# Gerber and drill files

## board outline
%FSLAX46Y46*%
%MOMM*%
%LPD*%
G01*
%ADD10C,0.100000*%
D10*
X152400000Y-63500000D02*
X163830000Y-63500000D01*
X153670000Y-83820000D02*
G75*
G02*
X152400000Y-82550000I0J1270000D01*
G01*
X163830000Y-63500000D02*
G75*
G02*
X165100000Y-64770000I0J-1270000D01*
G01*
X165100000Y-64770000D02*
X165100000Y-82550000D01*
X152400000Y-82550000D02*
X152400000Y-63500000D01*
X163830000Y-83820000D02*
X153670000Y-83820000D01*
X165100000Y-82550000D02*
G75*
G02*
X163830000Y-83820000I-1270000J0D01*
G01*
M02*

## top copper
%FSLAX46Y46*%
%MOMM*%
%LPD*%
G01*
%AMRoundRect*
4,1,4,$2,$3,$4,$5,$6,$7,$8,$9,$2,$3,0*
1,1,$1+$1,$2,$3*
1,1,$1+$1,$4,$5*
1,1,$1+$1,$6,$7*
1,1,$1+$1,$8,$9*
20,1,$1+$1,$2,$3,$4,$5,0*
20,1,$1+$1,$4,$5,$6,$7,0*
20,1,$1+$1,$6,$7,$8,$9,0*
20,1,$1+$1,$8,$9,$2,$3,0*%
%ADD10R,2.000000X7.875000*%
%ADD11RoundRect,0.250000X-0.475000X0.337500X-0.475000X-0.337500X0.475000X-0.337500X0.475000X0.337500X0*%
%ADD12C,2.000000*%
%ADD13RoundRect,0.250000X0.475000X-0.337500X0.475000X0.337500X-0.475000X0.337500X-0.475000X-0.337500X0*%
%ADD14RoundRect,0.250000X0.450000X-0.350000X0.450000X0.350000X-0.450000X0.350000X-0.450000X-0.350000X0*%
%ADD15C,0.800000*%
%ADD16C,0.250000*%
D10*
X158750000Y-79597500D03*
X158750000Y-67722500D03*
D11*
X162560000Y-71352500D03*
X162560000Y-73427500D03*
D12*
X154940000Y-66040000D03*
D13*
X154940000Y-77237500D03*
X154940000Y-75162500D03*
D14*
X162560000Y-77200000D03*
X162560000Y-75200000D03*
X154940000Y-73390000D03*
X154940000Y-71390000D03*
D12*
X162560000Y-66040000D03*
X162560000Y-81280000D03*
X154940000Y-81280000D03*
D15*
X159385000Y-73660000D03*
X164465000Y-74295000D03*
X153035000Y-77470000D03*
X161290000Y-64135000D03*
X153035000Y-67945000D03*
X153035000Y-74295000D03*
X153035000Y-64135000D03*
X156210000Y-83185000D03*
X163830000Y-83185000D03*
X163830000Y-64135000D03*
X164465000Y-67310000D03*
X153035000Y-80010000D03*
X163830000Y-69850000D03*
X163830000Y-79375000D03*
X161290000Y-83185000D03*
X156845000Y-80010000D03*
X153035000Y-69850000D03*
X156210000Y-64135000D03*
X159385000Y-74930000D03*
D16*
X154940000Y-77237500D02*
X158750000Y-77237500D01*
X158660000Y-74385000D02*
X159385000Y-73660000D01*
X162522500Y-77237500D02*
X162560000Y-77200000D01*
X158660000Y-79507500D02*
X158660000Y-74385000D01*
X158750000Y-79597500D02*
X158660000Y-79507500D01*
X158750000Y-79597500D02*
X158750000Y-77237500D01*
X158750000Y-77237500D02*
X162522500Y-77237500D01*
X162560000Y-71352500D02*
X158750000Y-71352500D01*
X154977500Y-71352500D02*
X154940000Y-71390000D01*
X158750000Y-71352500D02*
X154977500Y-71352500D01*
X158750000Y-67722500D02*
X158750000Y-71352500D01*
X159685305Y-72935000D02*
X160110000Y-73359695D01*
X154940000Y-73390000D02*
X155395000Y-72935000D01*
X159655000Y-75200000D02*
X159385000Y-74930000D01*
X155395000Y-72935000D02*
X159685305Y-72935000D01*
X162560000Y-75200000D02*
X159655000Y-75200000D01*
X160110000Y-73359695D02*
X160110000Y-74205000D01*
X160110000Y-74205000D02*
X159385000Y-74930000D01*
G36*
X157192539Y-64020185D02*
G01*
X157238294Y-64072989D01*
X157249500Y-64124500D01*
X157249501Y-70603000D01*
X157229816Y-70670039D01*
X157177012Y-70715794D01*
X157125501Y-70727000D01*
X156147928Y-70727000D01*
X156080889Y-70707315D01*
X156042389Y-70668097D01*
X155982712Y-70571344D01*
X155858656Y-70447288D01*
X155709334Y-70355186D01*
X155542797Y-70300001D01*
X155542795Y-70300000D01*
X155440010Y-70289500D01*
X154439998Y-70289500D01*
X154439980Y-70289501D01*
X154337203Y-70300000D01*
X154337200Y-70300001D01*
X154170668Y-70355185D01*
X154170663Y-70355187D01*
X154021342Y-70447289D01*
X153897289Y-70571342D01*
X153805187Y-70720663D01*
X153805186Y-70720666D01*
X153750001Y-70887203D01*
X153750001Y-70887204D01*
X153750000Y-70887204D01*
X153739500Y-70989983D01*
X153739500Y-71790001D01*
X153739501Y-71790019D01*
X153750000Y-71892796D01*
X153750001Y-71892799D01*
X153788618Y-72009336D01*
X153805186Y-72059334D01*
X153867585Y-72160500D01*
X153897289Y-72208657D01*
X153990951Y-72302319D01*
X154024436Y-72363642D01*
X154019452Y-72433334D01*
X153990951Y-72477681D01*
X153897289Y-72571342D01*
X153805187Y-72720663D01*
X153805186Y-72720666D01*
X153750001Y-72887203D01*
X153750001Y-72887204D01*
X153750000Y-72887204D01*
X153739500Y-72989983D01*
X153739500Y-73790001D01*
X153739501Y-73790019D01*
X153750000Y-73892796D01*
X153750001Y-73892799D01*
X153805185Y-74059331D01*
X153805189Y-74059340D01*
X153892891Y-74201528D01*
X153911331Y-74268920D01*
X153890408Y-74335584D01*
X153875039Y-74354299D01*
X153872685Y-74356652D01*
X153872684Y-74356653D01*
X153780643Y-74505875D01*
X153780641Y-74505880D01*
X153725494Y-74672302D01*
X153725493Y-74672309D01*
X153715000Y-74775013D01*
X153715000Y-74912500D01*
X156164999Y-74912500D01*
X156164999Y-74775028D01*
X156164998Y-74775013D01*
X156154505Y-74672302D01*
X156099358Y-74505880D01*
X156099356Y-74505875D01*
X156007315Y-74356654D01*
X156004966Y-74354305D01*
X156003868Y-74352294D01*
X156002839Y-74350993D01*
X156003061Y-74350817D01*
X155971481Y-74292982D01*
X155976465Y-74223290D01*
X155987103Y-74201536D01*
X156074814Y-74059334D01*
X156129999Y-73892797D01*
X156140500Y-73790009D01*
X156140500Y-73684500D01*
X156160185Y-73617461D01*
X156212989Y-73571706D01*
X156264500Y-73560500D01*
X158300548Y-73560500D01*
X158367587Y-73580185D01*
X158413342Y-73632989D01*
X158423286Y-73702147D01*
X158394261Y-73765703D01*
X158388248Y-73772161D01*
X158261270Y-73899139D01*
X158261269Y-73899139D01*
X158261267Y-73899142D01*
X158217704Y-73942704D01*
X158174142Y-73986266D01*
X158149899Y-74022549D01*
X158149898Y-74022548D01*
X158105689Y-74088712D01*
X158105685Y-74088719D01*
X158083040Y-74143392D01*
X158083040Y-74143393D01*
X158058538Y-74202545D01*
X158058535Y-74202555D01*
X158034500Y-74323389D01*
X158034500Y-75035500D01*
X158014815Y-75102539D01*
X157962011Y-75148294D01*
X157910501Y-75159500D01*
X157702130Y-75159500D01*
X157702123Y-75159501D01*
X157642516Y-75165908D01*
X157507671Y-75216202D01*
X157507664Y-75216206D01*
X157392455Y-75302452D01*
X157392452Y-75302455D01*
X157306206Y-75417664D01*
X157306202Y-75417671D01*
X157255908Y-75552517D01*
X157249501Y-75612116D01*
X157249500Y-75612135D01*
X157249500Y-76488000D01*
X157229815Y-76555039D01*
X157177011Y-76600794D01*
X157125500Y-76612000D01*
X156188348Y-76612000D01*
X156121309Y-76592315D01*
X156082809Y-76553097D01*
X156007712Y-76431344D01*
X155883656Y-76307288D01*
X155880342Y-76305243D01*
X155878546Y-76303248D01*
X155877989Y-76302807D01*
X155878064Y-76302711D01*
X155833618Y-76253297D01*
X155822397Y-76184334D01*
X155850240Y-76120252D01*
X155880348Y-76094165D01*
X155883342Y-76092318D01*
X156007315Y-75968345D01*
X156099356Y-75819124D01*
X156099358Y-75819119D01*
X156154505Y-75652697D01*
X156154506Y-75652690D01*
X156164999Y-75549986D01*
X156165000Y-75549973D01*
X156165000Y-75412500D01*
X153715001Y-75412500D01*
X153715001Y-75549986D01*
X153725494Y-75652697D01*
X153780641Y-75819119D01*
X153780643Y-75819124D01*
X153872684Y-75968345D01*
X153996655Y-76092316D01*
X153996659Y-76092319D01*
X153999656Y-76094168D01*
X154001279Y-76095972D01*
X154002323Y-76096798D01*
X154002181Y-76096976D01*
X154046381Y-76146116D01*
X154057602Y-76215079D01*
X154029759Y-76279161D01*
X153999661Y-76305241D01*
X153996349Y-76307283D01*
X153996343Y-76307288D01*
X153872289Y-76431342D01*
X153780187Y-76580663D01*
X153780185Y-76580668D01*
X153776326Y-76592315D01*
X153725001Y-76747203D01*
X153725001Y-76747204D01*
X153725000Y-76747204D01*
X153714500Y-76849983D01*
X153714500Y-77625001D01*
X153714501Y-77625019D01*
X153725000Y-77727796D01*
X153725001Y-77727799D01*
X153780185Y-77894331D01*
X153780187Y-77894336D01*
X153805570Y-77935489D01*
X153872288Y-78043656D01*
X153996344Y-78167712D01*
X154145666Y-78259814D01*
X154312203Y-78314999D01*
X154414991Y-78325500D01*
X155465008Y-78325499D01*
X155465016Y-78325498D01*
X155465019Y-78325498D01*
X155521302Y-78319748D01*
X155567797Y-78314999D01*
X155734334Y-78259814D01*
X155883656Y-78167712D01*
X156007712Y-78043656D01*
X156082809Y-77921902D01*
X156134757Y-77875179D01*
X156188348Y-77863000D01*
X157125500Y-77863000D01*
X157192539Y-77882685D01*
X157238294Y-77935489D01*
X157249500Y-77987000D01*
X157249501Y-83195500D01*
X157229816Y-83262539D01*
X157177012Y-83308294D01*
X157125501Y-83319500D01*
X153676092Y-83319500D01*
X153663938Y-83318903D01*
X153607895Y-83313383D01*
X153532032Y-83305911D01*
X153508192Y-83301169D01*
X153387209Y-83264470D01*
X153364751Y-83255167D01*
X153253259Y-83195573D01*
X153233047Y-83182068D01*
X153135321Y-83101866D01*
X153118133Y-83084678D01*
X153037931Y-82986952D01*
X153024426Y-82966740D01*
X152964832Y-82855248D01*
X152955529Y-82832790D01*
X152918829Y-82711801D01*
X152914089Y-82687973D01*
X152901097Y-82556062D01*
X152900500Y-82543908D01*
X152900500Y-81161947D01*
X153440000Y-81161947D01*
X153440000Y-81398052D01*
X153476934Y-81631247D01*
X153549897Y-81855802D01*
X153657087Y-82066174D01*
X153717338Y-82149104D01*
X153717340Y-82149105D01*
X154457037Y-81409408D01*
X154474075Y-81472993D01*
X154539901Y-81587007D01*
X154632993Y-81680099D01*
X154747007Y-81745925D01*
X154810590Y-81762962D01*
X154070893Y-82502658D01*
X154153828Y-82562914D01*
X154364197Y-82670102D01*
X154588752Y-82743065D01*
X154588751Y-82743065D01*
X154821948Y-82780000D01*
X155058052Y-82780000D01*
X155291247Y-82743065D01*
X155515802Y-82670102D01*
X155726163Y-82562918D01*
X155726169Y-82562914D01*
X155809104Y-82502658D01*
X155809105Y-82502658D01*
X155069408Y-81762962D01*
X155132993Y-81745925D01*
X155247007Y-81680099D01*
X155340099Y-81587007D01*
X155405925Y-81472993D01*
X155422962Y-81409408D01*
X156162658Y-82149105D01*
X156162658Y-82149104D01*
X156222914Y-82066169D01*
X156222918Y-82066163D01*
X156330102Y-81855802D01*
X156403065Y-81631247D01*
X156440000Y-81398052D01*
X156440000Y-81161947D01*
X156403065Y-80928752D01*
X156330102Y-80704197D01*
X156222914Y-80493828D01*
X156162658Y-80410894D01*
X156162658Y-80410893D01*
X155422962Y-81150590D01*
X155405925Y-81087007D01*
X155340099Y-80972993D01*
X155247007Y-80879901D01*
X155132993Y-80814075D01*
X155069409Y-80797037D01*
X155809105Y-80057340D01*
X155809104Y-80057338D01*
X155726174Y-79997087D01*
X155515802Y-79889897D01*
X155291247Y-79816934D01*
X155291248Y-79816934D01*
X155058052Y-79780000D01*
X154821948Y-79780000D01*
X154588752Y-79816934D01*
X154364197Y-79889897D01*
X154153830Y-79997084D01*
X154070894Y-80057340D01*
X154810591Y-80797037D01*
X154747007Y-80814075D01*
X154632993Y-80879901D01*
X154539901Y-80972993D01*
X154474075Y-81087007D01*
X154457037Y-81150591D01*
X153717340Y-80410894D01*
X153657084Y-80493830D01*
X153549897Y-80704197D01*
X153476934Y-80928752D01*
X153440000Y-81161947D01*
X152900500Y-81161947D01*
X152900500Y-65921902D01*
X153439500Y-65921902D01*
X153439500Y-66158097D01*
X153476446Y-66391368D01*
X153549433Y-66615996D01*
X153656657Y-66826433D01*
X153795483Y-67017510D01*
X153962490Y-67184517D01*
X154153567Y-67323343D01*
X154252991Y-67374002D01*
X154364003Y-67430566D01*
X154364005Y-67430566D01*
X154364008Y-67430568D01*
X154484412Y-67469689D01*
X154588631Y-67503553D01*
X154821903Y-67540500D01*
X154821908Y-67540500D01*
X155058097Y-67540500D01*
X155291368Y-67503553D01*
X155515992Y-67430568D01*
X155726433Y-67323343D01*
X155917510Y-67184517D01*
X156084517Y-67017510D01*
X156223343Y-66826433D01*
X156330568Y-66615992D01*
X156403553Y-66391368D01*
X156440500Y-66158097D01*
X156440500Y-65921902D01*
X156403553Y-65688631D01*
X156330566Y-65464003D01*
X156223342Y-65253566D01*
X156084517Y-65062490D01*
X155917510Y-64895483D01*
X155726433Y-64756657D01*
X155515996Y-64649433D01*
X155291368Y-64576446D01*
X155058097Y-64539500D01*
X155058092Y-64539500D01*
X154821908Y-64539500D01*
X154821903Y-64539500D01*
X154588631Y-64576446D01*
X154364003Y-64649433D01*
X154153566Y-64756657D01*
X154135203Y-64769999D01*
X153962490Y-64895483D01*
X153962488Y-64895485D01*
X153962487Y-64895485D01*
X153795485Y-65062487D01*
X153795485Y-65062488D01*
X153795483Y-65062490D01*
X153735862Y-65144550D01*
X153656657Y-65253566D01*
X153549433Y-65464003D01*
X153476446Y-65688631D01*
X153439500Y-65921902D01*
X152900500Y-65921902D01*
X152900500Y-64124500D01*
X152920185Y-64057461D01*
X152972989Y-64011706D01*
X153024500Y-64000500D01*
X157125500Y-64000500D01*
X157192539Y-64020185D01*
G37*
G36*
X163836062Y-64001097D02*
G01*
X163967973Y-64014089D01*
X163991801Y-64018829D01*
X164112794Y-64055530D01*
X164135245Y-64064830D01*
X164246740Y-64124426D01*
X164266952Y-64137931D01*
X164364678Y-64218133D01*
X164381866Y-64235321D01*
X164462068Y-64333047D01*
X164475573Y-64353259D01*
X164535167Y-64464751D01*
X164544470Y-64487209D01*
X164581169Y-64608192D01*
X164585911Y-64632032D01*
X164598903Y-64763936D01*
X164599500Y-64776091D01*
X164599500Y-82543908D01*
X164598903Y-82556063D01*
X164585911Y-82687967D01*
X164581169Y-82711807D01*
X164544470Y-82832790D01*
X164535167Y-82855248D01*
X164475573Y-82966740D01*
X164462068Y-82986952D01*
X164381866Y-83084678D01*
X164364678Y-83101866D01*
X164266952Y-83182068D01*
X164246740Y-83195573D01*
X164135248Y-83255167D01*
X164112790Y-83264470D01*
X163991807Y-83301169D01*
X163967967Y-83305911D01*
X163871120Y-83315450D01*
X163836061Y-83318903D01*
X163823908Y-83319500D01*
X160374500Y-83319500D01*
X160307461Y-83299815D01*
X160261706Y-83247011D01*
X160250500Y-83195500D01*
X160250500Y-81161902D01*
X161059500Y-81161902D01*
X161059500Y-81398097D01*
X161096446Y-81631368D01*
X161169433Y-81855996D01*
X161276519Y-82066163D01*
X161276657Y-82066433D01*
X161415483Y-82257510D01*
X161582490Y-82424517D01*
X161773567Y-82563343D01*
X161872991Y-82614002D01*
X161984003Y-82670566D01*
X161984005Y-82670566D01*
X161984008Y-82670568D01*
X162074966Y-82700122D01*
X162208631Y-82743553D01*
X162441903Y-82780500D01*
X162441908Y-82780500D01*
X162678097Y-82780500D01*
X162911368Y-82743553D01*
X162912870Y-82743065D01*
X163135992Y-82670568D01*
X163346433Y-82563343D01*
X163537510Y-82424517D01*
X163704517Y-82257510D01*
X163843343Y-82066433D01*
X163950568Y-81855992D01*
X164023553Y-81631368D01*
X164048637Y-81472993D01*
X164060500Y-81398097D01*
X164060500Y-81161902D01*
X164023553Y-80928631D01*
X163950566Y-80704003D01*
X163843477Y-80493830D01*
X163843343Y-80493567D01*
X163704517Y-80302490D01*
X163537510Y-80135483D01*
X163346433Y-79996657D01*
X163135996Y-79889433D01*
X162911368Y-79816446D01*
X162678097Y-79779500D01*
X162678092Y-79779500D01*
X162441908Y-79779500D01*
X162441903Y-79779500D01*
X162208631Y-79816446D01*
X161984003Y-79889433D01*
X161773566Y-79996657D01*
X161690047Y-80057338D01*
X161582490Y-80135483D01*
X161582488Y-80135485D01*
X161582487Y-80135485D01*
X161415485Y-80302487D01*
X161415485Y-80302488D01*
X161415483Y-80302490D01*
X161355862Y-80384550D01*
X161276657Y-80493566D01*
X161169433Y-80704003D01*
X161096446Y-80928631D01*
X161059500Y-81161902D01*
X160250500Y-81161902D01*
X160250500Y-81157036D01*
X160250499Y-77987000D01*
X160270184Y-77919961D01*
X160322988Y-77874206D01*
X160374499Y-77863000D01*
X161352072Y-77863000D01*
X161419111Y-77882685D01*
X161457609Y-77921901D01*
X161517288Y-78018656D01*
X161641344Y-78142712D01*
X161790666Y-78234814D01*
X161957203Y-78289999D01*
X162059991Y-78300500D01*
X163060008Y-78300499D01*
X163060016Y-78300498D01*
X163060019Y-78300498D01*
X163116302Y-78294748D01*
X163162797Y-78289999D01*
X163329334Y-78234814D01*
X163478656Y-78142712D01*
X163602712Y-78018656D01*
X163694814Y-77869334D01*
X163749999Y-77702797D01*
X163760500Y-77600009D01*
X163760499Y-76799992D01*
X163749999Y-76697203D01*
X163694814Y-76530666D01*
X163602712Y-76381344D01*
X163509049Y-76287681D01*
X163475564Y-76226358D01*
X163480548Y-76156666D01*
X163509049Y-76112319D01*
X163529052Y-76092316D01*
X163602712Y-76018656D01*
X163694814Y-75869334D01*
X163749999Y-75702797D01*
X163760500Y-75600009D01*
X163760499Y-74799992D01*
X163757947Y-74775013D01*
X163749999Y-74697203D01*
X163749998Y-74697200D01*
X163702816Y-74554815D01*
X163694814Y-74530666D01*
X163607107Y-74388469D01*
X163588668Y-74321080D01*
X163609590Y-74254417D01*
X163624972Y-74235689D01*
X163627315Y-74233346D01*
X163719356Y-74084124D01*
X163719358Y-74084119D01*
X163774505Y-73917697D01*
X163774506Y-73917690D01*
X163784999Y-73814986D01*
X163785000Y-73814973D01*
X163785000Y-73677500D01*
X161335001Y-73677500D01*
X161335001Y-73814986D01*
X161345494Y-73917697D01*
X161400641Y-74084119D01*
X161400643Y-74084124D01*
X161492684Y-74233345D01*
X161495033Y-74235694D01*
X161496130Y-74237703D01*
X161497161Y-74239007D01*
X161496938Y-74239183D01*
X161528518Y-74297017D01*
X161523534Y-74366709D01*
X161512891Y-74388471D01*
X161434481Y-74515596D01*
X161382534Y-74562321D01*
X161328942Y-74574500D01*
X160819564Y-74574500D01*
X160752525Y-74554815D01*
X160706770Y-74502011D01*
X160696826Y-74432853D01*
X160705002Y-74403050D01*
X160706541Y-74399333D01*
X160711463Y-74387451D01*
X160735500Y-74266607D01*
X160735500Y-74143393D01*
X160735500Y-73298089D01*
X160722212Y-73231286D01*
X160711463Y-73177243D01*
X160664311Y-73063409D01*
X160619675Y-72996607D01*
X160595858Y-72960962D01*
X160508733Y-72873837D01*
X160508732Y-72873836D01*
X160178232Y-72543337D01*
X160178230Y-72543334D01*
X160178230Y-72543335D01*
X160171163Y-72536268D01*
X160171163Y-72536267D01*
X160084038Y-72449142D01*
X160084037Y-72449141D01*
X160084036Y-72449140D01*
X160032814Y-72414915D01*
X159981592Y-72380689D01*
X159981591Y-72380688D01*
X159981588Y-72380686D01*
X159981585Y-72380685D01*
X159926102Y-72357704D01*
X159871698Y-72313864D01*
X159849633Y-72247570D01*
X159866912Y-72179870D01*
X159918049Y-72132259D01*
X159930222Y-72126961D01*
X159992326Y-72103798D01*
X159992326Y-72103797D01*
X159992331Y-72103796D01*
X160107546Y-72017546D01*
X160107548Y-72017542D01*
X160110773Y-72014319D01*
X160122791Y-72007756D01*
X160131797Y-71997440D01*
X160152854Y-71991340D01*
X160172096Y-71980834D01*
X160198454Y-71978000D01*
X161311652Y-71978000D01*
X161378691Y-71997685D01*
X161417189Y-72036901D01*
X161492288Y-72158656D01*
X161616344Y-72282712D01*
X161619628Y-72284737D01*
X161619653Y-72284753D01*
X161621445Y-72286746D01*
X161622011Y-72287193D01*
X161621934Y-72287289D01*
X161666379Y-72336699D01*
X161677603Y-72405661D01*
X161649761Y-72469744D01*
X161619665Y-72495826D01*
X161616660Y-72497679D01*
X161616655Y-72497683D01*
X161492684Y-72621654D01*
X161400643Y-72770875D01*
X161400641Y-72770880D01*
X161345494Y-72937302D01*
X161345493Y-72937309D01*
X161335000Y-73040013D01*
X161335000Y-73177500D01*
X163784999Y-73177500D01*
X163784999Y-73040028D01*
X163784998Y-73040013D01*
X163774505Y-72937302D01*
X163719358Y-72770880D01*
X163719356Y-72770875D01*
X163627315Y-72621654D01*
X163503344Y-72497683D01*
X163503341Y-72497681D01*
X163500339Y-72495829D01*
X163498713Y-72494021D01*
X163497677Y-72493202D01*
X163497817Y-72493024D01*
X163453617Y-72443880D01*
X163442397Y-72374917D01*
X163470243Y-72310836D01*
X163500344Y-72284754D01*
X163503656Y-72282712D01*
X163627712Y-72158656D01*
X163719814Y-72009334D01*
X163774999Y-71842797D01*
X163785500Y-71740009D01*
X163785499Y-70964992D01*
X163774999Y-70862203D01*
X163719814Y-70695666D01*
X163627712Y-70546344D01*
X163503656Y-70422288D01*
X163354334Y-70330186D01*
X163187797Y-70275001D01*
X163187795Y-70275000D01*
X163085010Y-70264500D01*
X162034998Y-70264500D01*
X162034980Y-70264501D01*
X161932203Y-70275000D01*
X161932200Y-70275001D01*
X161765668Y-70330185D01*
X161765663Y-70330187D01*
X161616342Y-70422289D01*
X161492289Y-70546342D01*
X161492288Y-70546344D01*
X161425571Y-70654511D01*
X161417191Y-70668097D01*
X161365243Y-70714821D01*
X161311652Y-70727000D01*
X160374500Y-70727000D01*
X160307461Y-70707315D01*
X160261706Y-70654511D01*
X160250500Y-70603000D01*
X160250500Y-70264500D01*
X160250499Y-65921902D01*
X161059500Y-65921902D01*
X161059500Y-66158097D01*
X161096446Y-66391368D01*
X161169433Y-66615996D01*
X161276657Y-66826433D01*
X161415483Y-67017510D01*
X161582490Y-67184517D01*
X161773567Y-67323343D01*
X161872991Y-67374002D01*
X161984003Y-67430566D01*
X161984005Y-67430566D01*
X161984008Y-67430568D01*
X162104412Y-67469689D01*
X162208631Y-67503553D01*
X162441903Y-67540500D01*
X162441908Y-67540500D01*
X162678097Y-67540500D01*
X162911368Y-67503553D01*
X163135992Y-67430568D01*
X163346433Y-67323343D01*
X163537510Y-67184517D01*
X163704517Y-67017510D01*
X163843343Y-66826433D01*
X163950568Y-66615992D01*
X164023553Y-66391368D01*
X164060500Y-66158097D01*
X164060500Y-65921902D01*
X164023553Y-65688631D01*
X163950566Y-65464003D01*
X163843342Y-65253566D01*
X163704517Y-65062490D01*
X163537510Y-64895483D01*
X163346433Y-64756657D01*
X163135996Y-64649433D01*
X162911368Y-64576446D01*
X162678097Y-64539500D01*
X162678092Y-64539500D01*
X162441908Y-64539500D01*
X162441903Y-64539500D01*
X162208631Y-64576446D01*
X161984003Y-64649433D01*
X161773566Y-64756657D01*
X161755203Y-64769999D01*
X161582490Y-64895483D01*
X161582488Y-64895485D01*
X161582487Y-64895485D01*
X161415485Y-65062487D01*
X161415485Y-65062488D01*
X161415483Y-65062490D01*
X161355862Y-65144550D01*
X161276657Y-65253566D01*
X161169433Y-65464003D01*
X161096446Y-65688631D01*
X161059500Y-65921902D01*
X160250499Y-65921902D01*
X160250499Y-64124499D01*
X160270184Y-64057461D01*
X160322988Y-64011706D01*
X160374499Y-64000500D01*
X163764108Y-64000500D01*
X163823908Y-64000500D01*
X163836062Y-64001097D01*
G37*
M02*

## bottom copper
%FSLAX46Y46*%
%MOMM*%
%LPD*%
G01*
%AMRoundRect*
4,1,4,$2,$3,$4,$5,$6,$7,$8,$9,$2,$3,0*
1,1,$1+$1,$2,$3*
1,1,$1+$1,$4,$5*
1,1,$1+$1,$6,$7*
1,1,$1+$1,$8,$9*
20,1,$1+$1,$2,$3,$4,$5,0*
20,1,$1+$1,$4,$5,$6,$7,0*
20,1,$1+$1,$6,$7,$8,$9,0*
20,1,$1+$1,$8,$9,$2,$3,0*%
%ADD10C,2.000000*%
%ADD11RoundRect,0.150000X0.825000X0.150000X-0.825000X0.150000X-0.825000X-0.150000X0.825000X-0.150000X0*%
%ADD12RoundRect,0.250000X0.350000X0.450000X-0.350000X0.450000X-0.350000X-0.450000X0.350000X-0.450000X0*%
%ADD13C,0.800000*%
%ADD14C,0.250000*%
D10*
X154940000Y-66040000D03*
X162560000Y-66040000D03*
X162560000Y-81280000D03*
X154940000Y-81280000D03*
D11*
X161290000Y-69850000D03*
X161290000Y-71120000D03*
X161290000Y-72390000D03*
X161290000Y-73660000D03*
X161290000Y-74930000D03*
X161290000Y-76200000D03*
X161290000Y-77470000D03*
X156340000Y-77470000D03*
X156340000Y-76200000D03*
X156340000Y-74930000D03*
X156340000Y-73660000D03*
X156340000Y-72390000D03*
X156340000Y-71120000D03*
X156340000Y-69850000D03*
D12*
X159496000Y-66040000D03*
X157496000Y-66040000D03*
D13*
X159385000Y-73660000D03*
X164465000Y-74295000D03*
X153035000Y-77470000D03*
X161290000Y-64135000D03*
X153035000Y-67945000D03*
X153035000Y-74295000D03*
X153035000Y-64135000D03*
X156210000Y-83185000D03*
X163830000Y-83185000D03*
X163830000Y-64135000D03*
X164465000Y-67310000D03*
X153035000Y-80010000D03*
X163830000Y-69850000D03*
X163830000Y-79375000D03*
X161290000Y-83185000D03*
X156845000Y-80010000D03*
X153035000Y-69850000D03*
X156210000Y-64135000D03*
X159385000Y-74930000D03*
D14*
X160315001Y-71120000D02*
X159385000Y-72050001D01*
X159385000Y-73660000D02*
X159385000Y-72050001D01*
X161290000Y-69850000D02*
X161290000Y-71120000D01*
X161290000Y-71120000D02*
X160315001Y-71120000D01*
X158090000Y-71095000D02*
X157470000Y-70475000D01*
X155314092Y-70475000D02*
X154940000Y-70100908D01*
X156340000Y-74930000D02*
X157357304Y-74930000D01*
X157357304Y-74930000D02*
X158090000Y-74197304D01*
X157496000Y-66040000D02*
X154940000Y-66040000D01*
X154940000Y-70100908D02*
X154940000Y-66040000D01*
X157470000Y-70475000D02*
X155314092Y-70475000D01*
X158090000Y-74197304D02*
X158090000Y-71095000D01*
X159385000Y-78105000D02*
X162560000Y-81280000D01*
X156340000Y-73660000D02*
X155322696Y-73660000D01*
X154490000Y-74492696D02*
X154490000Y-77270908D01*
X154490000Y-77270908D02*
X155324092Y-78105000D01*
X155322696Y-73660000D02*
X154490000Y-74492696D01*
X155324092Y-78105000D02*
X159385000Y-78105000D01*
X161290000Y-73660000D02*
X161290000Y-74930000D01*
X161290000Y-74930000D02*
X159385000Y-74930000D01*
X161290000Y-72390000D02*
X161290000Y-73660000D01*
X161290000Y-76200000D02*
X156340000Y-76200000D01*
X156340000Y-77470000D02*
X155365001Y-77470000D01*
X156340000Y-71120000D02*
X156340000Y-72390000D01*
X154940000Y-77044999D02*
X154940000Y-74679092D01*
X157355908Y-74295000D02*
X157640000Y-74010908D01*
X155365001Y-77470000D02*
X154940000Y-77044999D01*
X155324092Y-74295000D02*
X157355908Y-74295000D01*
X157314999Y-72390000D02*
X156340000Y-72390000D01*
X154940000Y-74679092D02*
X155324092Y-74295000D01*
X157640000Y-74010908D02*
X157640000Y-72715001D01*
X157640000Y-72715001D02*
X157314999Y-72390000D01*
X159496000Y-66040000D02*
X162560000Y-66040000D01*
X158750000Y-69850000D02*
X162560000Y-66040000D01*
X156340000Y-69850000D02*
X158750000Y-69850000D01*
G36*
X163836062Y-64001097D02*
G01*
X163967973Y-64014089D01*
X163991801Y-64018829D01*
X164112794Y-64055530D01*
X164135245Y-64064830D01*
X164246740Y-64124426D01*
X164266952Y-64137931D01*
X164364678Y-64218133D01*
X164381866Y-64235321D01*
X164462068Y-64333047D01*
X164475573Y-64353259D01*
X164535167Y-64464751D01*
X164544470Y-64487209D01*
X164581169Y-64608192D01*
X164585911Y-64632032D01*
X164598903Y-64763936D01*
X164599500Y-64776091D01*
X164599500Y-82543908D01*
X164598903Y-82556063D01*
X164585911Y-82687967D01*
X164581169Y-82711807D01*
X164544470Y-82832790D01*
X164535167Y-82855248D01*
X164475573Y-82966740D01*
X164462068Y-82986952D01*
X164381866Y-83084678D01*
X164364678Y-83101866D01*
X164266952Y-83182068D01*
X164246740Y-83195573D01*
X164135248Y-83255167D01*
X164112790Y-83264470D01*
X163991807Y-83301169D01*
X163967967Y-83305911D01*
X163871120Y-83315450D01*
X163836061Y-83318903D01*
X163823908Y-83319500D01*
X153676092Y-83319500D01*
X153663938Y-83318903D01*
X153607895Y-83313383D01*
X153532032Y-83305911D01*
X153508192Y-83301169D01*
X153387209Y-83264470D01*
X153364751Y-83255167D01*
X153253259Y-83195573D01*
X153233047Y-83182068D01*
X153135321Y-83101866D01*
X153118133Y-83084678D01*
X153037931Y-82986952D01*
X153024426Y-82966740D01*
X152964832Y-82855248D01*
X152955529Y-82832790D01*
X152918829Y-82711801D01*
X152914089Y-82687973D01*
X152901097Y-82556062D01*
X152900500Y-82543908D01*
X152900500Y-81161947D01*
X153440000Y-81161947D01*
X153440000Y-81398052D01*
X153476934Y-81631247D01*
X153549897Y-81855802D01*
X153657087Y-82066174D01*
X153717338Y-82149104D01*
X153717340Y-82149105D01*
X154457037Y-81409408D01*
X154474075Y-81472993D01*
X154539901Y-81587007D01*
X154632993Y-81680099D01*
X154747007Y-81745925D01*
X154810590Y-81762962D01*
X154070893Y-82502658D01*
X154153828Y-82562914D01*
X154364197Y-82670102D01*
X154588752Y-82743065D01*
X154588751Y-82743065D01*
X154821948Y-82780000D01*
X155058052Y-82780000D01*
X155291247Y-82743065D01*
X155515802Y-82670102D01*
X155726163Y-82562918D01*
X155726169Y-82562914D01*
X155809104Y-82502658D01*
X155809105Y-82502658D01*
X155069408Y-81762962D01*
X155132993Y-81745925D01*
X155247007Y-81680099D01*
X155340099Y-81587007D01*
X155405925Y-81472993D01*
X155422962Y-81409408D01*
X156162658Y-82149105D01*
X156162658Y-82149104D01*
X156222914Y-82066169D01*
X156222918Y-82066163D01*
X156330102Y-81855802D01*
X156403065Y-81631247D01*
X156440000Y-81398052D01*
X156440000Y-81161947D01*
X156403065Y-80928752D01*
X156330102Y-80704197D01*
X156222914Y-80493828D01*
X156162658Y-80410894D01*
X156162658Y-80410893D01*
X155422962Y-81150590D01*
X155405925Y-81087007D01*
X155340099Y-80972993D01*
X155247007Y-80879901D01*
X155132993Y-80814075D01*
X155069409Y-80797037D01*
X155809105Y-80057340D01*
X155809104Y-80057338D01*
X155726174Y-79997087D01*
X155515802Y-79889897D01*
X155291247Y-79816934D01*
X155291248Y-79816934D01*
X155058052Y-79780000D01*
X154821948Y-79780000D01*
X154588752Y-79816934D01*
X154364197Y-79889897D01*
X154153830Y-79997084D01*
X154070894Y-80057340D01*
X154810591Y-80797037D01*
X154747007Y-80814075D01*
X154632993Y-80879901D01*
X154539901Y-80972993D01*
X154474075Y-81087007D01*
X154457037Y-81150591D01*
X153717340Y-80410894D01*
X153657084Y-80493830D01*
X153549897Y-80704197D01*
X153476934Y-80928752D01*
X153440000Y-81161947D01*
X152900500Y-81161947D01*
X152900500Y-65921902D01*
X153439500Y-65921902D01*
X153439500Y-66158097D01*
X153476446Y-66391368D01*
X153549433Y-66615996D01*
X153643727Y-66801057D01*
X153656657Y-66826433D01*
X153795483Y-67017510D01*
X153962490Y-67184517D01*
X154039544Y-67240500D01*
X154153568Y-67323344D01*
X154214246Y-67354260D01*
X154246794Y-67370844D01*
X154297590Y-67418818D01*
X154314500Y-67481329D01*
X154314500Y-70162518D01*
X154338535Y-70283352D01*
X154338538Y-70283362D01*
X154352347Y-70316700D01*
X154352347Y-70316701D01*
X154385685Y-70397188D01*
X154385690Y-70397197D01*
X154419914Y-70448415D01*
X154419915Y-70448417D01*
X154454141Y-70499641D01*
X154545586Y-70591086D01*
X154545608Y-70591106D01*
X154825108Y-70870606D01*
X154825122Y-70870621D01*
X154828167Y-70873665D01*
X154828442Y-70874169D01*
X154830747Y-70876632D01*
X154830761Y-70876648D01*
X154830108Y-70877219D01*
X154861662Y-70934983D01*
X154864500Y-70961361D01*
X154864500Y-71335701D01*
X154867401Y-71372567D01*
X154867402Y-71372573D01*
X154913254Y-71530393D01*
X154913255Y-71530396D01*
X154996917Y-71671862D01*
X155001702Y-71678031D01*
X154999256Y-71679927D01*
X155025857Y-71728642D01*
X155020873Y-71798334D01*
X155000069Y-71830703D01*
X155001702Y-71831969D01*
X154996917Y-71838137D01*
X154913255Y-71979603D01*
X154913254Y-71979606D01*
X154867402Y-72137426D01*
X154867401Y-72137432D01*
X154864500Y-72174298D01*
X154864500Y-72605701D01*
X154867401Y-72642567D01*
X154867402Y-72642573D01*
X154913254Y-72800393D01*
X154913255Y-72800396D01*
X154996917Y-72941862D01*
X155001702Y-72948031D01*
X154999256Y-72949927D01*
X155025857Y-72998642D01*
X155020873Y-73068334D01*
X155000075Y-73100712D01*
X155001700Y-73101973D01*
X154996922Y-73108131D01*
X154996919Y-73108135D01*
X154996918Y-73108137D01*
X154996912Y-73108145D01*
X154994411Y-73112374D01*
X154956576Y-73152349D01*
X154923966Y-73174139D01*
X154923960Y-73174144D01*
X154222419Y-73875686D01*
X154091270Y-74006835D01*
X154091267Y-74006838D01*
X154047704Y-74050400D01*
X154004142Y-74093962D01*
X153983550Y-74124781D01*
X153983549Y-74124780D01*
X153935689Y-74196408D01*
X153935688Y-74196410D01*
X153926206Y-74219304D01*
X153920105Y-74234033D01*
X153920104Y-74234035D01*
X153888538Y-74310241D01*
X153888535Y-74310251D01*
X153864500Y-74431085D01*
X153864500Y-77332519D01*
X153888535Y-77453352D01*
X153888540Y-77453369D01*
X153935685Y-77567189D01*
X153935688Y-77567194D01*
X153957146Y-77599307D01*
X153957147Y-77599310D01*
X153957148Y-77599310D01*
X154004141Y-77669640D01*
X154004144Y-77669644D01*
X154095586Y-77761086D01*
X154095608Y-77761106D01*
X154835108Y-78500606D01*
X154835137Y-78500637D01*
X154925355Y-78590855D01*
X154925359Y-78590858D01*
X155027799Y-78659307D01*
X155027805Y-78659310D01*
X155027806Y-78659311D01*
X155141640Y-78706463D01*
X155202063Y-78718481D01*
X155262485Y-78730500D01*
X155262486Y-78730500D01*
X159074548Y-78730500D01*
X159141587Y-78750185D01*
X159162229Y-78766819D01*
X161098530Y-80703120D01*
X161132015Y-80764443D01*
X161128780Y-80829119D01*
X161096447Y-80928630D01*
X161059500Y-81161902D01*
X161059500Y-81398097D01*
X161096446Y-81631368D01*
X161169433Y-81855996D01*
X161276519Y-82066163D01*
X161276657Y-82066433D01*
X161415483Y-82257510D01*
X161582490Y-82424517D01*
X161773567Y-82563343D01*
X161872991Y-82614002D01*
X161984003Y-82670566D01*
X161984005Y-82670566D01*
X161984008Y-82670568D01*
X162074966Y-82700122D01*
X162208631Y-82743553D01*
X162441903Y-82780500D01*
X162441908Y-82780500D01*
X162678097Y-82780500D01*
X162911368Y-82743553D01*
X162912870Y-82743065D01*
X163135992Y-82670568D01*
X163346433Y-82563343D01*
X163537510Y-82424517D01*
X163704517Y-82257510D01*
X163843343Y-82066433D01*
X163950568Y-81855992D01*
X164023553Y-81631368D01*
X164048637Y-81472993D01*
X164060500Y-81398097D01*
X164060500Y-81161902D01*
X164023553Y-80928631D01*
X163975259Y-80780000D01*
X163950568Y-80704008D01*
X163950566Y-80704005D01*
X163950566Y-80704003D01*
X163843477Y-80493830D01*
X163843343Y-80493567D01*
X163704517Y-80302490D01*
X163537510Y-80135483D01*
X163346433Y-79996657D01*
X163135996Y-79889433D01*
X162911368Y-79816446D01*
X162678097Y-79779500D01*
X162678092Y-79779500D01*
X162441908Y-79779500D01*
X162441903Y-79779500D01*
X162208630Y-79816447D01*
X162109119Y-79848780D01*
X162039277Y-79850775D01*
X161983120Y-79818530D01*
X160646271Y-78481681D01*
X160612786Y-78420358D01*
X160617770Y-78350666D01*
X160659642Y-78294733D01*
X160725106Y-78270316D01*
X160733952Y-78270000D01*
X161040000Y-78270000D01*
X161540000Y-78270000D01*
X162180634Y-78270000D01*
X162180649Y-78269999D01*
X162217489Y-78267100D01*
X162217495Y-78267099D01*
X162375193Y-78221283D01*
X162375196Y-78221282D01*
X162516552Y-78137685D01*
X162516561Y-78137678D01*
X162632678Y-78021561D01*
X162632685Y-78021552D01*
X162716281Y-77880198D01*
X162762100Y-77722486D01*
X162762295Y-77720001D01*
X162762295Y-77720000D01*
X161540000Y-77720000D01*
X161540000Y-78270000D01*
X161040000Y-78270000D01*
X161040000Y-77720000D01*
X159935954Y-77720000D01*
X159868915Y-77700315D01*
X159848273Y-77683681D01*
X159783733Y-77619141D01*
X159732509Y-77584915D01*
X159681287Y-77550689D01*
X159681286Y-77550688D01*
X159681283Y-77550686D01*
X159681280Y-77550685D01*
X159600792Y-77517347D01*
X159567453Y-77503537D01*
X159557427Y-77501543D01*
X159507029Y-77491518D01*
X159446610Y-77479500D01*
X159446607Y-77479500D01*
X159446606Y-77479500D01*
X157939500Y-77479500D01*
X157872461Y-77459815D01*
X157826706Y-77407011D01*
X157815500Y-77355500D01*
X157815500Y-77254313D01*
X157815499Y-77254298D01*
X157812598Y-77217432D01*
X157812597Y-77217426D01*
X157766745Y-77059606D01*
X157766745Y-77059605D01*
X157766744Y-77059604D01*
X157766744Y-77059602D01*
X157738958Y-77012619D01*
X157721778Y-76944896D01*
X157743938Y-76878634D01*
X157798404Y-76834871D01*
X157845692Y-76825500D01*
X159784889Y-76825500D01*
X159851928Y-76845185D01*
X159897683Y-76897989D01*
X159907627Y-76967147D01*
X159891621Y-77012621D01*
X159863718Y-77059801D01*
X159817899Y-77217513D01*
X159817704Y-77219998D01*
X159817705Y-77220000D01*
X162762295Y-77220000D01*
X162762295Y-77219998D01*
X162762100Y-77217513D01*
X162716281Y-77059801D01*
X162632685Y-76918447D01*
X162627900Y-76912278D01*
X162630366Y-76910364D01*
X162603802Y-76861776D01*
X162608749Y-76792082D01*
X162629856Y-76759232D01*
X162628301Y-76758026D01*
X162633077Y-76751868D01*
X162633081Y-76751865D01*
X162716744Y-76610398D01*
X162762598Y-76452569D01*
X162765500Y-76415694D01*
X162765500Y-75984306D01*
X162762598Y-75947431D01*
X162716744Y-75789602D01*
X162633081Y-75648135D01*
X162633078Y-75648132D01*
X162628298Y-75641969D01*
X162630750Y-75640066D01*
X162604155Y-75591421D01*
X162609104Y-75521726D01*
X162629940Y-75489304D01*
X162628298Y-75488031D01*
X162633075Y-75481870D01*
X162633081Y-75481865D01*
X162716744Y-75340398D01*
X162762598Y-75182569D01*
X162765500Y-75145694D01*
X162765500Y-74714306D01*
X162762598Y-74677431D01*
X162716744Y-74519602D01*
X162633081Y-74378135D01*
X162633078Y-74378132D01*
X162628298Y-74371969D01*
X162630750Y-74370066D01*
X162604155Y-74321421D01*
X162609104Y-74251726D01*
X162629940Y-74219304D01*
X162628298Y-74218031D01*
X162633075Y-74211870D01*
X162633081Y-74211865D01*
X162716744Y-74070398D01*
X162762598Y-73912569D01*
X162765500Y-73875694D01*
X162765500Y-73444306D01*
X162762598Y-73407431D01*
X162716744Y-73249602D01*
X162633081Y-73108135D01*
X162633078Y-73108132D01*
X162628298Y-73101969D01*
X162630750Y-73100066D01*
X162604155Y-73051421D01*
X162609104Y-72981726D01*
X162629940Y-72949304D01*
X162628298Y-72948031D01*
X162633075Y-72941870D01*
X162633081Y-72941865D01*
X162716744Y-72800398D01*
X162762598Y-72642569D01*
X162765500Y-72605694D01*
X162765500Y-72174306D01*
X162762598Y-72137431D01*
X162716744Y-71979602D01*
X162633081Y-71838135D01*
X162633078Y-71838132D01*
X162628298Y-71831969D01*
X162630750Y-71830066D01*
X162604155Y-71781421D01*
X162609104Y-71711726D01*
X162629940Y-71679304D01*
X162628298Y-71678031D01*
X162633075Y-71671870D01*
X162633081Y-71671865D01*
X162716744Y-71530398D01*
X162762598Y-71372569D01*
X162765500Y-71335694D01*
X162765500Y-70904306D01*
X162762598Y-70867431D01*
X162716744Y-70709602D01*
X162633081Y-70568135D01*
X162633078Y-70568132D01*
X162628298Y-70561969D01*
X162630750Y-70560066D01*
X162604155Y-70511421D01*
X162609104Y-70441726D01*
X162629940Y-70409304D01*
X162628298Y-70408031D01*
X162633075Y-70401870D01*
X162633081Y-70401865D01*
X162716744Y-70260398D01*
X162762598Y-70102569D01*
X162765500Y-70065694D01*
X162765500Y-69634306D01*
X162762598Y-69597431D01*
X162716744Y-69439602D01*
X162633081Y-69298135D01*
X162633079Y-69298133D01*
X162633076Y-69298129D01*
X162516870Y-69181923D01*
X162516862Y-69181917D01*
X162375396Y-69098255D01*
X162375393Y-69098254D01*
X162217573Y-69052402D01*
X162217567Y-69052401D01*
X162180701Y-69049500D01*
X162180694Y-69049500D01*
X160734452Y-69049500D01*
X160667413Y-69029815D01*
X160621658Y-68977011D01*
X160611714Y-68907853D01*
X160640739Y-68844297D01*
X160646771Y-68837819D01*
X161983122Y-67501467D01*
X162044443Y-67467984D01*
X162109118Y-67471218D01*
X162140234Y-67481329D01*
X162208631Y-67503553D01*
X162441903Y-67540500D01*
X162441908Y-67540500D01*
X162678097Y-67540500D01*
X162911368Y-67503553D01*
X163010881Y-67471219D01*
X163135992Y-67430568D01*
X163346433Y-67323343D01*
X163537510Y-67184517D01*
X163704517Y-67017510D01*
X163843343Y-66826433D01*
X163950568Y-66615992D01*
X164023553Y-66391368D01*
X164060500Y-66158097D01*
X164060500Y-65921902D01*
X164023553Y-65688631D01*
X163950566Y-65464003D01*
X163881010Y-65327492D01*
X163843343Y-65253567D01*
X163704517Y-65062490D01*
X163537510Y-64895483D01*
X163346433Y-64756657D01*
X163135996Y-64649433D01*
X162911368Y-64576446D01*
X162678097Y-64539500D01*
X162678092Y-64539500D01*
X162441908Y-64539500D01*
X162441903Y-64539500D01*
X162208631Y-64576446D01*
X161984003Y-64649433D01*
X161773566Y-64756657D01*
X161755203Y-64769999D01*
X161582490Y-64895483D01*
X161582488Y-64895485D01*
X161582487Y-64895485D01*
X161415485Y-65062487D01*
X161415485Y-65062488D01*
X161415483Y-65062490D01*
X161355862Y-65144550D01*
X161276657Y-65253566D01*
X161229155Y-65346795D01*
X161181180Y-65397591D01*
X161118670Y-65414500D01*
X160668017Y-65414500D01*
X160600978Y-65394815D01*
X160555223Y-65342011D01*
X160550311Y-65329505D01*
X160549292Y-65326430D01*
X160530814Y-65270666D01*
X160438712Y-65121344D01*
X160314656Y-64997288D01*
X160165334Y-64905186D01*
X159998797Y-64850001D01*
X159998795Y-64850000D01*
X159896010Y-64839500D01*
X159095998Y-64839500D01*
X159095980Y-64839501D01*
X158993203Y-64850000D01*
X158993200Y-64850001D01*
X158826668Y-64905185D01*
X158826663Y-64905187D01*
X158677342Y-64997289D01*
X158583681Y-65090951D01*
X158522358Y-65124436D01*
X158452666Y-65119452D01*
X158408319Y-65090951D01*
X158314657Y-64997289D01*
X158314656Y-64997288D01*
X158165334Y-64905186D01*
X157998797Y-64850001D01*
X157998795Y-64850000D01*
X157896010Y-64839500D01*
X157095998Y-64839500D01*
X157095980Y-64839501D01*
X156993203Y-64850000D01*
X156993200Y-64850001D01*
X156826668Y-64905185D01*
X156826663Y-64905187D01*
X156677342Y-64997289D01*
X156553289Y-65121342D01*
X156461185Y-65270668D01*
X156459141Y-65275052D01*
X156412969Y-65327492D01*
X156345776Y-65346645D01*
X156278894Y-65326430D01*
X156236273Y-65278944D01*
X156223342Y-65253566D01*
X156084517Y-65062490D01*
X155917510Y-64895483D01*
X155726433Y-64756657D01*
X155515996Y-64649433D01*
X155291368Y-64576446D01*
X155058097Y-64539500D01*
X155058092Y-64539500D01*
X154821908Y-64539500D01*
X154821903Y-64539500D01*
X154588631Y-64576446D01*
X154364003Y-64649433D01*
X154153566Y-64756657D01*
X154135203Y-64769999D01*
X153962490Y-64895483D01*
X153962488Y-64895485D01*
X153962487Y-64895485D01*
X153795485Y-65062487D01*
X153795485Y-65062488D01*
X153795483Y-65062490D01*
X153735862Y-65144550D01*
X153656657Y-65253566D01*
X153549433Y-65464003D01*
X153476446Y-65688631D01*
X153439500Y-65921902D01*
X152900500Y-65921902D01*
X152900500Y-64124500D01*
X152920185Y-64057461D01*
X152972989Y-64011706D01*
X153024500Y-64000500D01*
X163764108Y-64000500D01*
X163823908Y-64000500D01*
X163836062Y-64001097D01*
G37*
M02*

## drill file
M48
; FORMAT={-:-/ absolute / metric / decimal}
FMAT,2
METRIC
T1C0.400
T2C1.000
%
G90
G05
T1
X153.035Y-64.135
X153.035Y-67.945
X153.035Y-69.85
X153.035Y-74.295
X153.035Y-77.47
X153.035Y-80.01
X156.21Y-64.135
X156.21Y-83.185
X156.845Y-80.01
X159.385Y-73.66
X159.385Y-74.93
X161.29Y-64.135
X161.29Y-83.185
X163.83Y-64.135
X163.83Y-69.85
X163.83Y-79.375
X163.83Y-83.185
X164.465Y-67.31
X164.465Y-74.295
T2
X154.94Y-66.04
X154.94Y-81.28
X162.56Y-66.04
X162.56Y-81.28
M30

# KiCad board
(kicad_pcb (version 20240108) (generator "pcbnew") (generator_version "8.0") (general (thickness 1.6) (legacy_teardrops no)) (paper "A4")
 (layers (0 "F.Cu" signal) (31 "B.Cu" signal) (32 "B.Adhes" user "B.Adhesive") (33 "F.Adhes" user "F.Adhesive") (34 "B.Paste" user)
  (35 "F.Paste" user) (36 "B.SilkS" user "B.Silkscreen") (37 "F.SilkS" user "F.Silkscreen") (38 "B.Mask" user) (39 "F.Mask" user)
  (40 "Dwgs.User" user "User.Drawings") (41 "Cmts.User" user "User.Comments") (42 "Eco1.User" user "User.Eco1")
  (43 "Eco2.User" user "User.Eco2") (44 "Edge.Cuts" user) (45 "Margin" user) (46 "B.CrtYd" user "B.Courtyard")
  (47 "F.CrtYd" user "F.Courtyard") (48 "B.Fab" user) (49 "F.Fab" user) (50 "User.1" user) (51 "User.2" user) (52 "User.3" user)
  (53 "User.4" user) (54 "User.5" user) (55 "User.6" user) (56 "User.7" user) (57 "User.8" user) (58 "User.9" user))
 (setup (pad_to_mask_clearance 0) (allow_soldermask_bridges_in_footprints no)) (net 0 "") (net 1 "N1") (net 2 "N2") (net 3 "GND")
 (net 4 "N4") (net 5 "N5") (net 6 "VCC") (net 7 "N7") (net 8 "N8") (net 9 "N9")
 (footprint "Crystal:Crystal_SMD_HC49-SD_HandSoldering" (layer "F.Cu") (at 158.75 73.66 90)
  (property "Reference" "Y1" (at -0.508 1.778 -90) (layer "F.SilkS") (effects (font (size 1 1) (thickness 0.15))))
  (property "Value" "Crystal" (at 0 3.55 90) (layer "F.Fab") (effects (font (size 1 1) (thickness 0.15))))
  (pad "1" smd rect (at -5.9375 0 90) (size 7.875 2) (layers "F.Cu" "F.Paste" "F.Mask") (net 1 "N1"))
  (pad "2" smd rect (at 5.9375 0 90) (size 7.875 2) (layers "F.Cu" "F.Paste" "F.Mask") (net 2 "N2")))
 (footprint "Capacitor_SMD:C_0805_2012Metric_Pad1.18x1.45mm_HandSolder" (layer "F.Cu") (at 162.56 72.39 -90)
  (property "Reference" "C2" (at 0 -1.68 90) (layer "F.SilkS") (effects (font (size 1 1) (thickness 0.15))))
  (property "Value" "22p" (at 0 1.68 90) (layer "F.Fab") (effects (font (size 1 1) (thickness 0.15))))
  (pad "1" smd roundrect (at -1.0375 0 270) (size 1.175 1.45) (layers "F.Cu" "F.Paste" "F.Mask") (roundrect_rratio 0.2127659574)
   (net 2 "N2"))
  (pad "2" smd roundrect (at 1.0375 0 270) (size 1.175 1.45) (layers "F.Cu" "F.Paste" "F.Mask") (roundrect_rratio 0.2127659574)
   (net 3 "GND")))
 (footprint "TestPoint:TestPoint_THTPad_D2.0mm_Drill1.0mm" (layer "F.Cu") (at 154.94 66.04)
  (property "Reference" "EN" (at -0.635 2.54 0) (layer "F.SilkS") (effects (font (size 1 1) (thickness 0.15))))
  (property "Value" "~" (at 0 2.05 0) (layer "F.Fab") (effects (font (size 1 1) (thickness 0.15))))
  (pad "1" thru_hole circle (at 0 0) (size 2 2) (drill 1) (layers "*.Cu" "*.Mask") (remove_unused_layers no) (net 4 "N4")))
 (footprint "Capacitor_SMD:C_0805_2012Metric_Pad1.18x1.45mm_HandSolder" (layer "F.Cu") (at 154.94 76.2 90)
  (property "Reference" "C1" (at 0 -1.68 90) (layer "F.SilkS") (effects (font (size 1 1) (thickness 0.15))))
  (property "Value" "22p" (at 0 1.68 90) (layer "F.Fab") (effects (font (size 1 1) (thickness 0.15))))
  (pad "1" smd roundrect (at -1.0375 0 90) (size 1.175 1.45) (layers "F.Cu" "F.Paste" "F.Mask") (roundrect_rratio 0.2127659574) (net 1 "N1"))
  (pad "2" smd roundrect (at 1.0375 0 90) (size 1.175 1.45) (layers "F.Cu" "F.Paste" "F.Mask") (roundrect_rratio 0.2127659574) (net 3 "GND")))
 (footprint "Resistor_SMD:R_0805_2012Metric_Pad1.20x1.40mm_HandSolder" (layer "F.Cu") (at 162.56 76.2 90)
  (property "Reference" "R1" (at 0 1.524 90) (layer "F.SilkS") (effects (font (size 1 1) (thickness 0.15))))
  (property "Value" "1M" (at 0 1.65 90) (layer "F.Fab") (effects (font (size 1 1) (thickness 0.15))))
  (pad "1" smd roundrect (at -1 0 90) (size 1.2 1.4) (layers "F.Cu" "F.Paste" "F.Mask") (roundrect_rratio 0.2083333333) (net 1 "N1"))
  (pad "2" smd roundrect (at 1 0 90) (size 1.2 1.4) (layers "F.Cu" "F.Paste" "F.Mask") (roundrect_rratio 0.2083333333) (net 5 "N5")))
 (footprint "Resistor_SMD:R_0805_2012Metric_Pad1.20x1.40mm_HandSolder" (layer "F.Cu") (at 154.94 72.39 90)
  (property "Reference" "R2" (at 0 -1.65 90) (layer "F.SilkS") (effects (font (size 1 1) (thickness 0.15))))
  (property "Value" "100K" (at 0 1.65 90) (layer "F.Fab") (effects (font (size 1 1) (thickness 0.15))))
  (pad "1" smd roundrect (at -1 0 90) (size 1.2 1.4) (layers "F.Cu" "F.Paste" "F.Mask") (roundrect_rratio 0.2083333333) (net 5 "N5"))
  (pad "2" smd roundrect (at 1 0 90) (size 1.2 1.4) (layers "F.Cu" "F.Paste" "F.Mask") (roundrect_rratio 0.2083333333) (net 2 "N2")))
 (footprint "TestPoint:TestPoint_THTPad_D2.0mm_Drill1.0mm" (layer "F.Cu") (at 162.56 66.04)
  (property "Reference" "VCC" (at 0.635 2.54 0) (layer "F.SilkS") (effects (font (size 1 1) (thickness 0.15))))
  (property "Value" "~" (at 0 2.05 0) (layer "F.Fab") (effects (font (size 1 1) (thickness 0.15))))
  (pad "1" thru_hole circle (at 0 0) (size 2 2) (drill 1) (layers "*.Cu" "*.Mask") (remove_unused_layers no) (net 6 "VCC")))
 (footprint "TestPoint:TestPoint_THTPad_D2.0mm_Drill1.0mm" (layer "F.Cu") (at 162.56 81.28)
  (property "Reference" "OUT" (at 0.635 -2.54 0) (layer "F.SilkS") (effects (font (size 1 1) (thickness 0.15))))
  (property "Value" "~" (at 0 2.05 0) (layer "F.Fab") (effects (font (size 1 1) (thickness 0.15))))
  (pad "1" thru_hole circle (at 0 0) (size 2 2) (drill 1) (layers "*.Cu" "*.Mask") (remove_unused_layers no) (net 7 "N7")))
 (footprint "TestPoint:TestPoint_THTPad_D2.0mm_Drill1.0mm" (layer "F.Cu") (at 154.94 81.28)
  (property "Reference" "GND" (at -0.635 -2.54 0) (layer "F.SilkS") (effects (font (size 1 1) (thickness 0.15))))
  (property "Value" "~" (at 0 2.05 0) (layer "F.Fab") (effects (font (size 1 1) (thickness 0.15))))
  (pad "1" thru_hole circle (at 0 0) (size 2 2) (drill 1) (layers "*.Cu" "*.Mask") (remove_unused_layers no) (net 3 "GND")))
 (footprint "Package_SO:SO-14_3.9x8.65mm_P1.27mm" (layer "B.Cu") (at 158.815 73.66 180)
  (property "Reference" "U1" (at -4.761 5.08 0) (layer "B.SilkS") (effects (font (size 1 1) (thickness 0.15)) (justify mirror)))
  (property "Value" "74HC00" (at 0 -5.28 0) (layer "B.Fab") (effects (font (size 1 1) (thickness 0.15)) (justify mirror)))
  (pad "1" smd roundrect (at -2.475 3.81 180) (size 1.95 0.6) (layers "B.Cu" "B.Paste" "B.Mask") (roundrect_rratio 0.25) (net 1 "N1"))
  (pad "2" smd roundrect (at -2.475 2.54 180) (size 1.95 0.6) (layers "B.Cu" "B.Paste" "B.Mask") (roundrect_rratio 0.25) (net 1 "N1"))
  (pad "3" smd roundrect (at -2.475 1.27 180) (size 1.95 0.6) (layers "B.Cu" "B.Paste" "B.Mask") (roundrect_rratio 0.25) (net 5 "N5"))
  (pad "4" smd roundrect (at -2.475 0 180) (size 1.95 0.6) (layers "B.Cu" "B.Paste" "B.Mask") (roundrect_rratio 0.25) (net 5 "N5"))
  (pad "5" smd roundrect (at -2.475 -1.27 180) (size 1.95 0.6) (layers "B.Cu" "B.Paste" "B.Mask") (roundrect_rratio 0.25) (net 5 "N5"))
  (pad "6" smd roundrect (at -2.475 -2.54 180) (size 1.95 0.6) (layers "B.Cu" "B.Paste" "B.Mask") (roundrect_rratio 0.25) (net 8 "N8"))
  (pad "7" smd roundrect (at -2.475 -3.81 180) (size 1.95 0.6) (layers "B.Cu" "B.Paste" "B.Mask") (roundrect_rratio 0.25) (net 3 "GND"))
  (pad "8" smd roundrect (at 2.475 -3.81 180) (size 1.95 0.6) (layers "B.Cu" "B.Paste" "B.Mask") (roundrect_rratio 0.25) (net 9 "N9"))
  (pad "9" smd roundrect (at 2.475 -2.54 180) (size 1.95 0.6) (layers "B.Cu" "B.Paste" "B.Mask") (roundrect_rratio 0.25) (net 8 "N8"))
  (pad "10" smd roundrect (at 2.475 -1.27 180) (size 1.95 0.6) (layers "B.Cu" "B.Paste" "B.Mask") (roundrect_rratio 0.25) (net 4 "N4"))
  (pad "11" smd roundrect (at 2.475 0 180) (size 1.95 0.6) (layers "B.Cu" "B.Paste" "B.Mask") (roundrect_rratio 0.25) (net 7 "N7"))
  (pad "12" smd roundrect (at 2.475 1.27 180) (size 1.95 0.6) (layers "B.Cu" "B.Paste" "B.Mask") (roundrect_rratio 0.25) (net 9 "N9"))
  (pad "13" smd roundrect (at 2.475 2.54 180) (size 1.95 0.6) (layers "B.Cu" "B.Paste" "B.Mask") (roundrect_rratio 0.25) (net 9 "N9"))
  (pad "14" smd roundrect (at 2.475 3.81 180) (size 1.95 0.6) (layers "B.Cu" "B.Paste" "B.Mask") (roundrect_rratio 0.25) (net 6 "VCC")))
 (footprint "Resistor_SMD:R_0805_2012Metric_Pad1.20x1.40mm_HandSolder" (layer "B.Cu") (at 158.496 66.04 180)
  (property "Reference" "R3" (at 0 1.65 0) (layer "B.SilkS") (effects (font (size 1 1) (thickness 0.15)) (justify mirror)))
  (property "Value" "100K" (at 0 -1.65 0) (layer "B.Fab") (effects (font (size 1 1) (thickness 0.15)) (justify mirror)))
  (pad "1" smd roundrect (at -1 0 180) (size 1.2 1.4) (layers "B.Cu" "B.Paste" "B.Mask") (roundrect_rratio 0.2083333333) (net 6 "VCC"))
  (pad "2" smd roundrect (at 1 0 180) (size 1.2 1.4) (layers "B.Cu" "B.Paste" "B.Mask") (roundrect_rratio 0.2083333333) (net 4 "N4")))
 (gr_line (start 152.4 63.5) (end 163.83 63.5) (stroke (width 0.1) (type default)) (layer "Edge.Cuts"))
 (gr_arc (start 153.67 83.82) (mid 152.771974 83.448026) (end 152.4 82.55) (stroke (width 0.1) (type default)) (layer "Edge.Cuts"))
 (gr_arc (start 163.83 63.5) (mid 164.728026 63.871974) (end 165.1 64.77) (stroke (width 0.1) (type default)) (layer "Edge.Cuts"))
 (gr_line (start 165.1 64.77) (end 165.1 82.55) (stroke (width 0.1) (type default)) (layer "Edge.Cuts"))
 (gr_line (start 152.4 82.55) (end 152.4 63.5) (stroke (width 0.1) (type default)) (layer "Edge.Cuts"))
 (gr_line (start 163.83 83.82) (end 153.67 83.82) (stroke (width 0.1) (type default)) (layer "Edge.Cuts"))
 (gr_arc (start 165.1 82.55) (mid 164.728026 83.448026) (end 163.83 83.82) (stroke (width 0.1) (type default)) (layer "Edge.Cuts"))
 (segment (start 154.94 77.2375) (end 158.75 77.2375) (width 0.25) (layer "F.Cu") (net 1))
 (segment (start 158.66 74.385) (end 159.385 73.66) (width 0.25) (layer "F.Cu") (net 1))
 (segment (start 162.5225 77.2375) (end 162.56 77.2) (width 0.25) (layer "F.Cu") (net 1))
 (segment (start 158.66 79.5075) (end 158.66 74.385) (width 0.25) (layer "F.Cu") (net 1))
 (segment (start 158.75 79.5975) (end 158.66 79.5075) (width 0.25) (layer "F.Cu") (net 1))
 (segment (start 158.75 79.5975) (end 158.75 77.2375) (width 0.25) (layer "F.Cu") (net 1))
 (segment (start 158.75 77.2375) (end 162.5225 77.2375) (width 0.25) (layer "F.Cu") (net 1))
 (via (at 159.385 73.66) (size 0.8) (drill 0.4) (layers "F.Cu" "B.Cu") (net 1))
 (segment (start 160.315001 71.12) (end 159.385 72.050001) (width 0.25) (layer "B.Cu") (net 1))
 (segment (start 159.385 73.66) (end 159.385 72.050001) (width 0.25) (layer "B.Cu") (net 1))
 (segment (start 161.29 69.85) (end 161.29 71.12) (width 0.25) (layer "B.Cu") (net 1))
 (segment (start 161.29 71.12) (end 160.315001 71.12) (width 0.25) (layer "B.Cu") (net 1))
 (via (at 164.465 74.295) (size 0.8) (drill 0.4) (layers "F.Cu" "B.Cu") (free yes) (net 3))
 (via (at 153.035 77.47) (size 0.8) (drill 0.4) (layers "F.Cu" "B.Cu") (free yes) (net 3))
 (via (at 161.29 64.135) (size 0.8) (drill 0.4) (layers "F.Cu" "B.Cu") (free yes) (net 3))
 (via (at 153.035 67.945) (size 0.8) (drill 0.4) (layers "F.Cu" "B.Cu") (free yes) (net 3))
 (via (at 153.035 74.295) (size 0.8) (drill 0.4) (layers "F.Cu" "B.Cu") (free yes) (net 3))
 (via (at 153.035 64.135) (size 0.8) (drill 0.4) (layers "F.Cu" "B.Cu") (free yes) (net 3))
 (via (at 156.21 83.185) (size 0.8) (drill 0.4) (layers "F.Cu" "B.Cu") (free yes) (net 3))
 (via (at 163.83 83.185) (size 0.8) (drill 0.4) (layers "F.Cu" "B.Cu") (free yes) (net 3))
 (via (at 163.83 64.135) (size 0.8) (drill 0.4) (layers "F.Cu" "B.Cu") (free yes) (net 3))
 (via (at 164.465 67.31) (size 0.8) (drill 0.4) (layers "F.Cu" "B.Cu") (free yes) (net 3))
 (via (at 153.035 80.01) (size 0.8) (drill 0.4) (layers "F.Cu" "B.Cu") (free yes) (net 3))
 (via (at 163.83 69.85) (size 0.8) (drill 0.4) (layers "F.Cu" "B.Cu") (free yes) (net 3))
 (via (at 163.83 79.375) (size 0.8) (drill 0.4) (layers "F.Cu" "B.Cu") (free yes) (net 3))
 (via (at 161.29 83.185) (size 0.8) (drill 0.4) (layers "F.Cu" "B.Cu") (free yes) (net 3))
 (via (at 156.845 80.01) (size 0.8) (drill 0.4) (layers "F.Cu" "B.Cu") (free yes) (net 3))
 (via (at 153.035 69.85) (size 0.8) (drill 0.4) (layers "F.Cu" "B.Cu") (free yes) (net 3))
 (via (at 156.21 64.135) (size 0.8) (drill 0.4) (layers "F.Cu" "B.Cu") (free yes) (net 3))
 (segment (start 162.56 71.3525) (end 158.75 71.3525) (width 0.25) (layer "F.Cu") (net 2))
 (segment (start 154.9775 71.3525) (end 154.94 71.39) (width 0.25) (layer "F.Cu") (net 2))
 (segment (start 158.75 71.3525) (end 154.9775 71.3525) (width 0.25) (layer "F.Cu") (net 2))
 (segment (start 158.75 67.7225) (end 158.75 71.3525) (width 0.25) (layer "F.Cu") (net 2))
 (segment (start 158.09 71.095) (end 157.47 70.475) (width 0.25) (layer "B.Cu") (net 4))
 (segment (start 155.314092 70.475) (end 154.94 70.100908) (width 0.25) (layer "B.Cu") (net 4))
 (segment (start 156.34 74.93) (end 157.357304 74.93) (width 0.25) (layer "B.Cu") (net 4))
 (segment (start 157.357304 74.93) (end 158.09 74.197304) (width 0.25) (layer "B.Cu") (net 4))
 (segment (start 157.496 66.04) (end 154.94 66.04) (width 0.25) (layer "B.Cu") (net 4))
 (segment (start 154.94 70.100908) (end 154.94 66.04) (width 0.25) (layer "B.Cu") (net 4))
 (segment (start 157.47 70.475) (end 155.314092 70.475) (width 0.25) (layer "B.Cu") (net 4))
 (segment (start 158.09 74.197304) (end 158.09 71.095) (width 0.25) (layer "B.Cu") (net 4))
 (segment (start 159.385 78.105) (end 162.56 81.28) (width 0.25) (layer "B.Cu") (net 7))
 (segment (start 156.34 73.66) (end 155.322696 73.66) (width 0.25) (layer "B.Cu") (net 7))
 (segment (start 154.49 74.492696) (end 154.49 77.270908) (width 0.25) (layer "B.Cu") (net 7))
 (segment (start 154.49 77.270908) (end 155.324092 78.105) (width 0.25) (layer "B.Cu") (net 7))
 (segment (start 155.322696 73.66) (end 154.49 74.492696) (width 0.25) (layer "B.Cu") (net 7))
 (segment (start 155.324092 78.105) (end 159.385 78.105) (width 0.25) (layer "B.Cu") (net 7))
 (segment (start 159.685305 72.935) (end 160.11 73.359695) (width 0.25) (layer "F.Cu") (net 5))
 (segment (start 154.94 73.39) (end 155.395 72.935) (width 0.25) (layer "F.Cu") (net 5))
 (segment (start 159.655 75.2) (end 159.385 74.93) (width 0.25) (layer "F.Cu") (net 5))
 (segment (start 155.395 72.935) (end 159.685305 72.935) (width 0.25) (layer "F.Cu") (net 5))
 (segment (start 162.56 75.2) (end 159.655 75.2) (width 0.25) (layer "F.Cu") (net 5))
 (segment (start 160.11 73.359695) (end 160.11 74.205) (width 0.25) (layer "F.Cu") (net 5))
 (segment (start 160.11 74.205) (end 159.385 74.93) (width 0.25) (layer "F.Cu") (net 5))
 (via (at 159.385 74.93) (size 0.8) (drill 0.4) (layers "F.Cu" "B.Cu") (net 5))
 (segment (start 161.29 73.66) (end 161.29 74.93) (width 0.25) (layer "B.Cu") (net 5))
 (segment (start 161.29 74.93) (end 159.385 74.93) (width 0.25) (layer "B.Cu") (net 5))
 (segment (start 161.29 72.39) (end 161.29 73.66) (width 0.25) (layer "B.Cu") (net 5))
 (segment (start 161.29 76.2) (end 156.34 76.2) (width 0.25) (layer "B.Cu") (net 8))
 (segment (start 156.34 77.47) (end 155.365001 77.47) (width 0.25) (layer "B.Cu") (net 9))
 (segment (start 156.34 71.12) (end 156.34 72.39) (width 0.25) (layer "B.Cu") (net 9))
 (segment (start 154.94 77.044999) (end 154.94 74.679092) (width 0.25) (layer "B.Cu") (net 9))
 (segment (start 157.355908 74.295) (end 157.64 74.010908) (width 0.25) (layer "B.Cu") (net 9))
 (segment (start 155.365001 77.47) (end 154.94 77.044999) (width 0.25) (layer "B.Cu") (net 9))
 (segment (start 155.324092 74.295) (end 157.355908 74.295) (width 0.25) (layer "B.Cu") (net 9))
 (segment (start 157.314999 72.39) (end 156.34 72.39) (width 0.25) (layer "B.Cu") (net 9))
 (segment (start 154.94 74.679092) (end 155.324092 74.295) (width 0.25) (layer "B.Cu") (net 9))
 (segment (start 157.64 74.010908) (end 157.64 72.715001) (width 0.25) (layer "B.Cu") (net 9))
 (segment (start 157.64 72.715001) (end 157.314999 72.39) (width 0.25) (layer "B.Cu") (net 9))
 (segment (start 159.496 66.04) (end 162.56 66.04) (width 0.25) (layer "B.Cu") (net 6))
 (segment (start 158.75 69.85) (end 162.56 66.04) (width 0.25) (layer "B.Cu") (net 6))
 (segment (start 156.34 69.85) (end 158.75 69.85) (width 0.25) (layer "B.Cu") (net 6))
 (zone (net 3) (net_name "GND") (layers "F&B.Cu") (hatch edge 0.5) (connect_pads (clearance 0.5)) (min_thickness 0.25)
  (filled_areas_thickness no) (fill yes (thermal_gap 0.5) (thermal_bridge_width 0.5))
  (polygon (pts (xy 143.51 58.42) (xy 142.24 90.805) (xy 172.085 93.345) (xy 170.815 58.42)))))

